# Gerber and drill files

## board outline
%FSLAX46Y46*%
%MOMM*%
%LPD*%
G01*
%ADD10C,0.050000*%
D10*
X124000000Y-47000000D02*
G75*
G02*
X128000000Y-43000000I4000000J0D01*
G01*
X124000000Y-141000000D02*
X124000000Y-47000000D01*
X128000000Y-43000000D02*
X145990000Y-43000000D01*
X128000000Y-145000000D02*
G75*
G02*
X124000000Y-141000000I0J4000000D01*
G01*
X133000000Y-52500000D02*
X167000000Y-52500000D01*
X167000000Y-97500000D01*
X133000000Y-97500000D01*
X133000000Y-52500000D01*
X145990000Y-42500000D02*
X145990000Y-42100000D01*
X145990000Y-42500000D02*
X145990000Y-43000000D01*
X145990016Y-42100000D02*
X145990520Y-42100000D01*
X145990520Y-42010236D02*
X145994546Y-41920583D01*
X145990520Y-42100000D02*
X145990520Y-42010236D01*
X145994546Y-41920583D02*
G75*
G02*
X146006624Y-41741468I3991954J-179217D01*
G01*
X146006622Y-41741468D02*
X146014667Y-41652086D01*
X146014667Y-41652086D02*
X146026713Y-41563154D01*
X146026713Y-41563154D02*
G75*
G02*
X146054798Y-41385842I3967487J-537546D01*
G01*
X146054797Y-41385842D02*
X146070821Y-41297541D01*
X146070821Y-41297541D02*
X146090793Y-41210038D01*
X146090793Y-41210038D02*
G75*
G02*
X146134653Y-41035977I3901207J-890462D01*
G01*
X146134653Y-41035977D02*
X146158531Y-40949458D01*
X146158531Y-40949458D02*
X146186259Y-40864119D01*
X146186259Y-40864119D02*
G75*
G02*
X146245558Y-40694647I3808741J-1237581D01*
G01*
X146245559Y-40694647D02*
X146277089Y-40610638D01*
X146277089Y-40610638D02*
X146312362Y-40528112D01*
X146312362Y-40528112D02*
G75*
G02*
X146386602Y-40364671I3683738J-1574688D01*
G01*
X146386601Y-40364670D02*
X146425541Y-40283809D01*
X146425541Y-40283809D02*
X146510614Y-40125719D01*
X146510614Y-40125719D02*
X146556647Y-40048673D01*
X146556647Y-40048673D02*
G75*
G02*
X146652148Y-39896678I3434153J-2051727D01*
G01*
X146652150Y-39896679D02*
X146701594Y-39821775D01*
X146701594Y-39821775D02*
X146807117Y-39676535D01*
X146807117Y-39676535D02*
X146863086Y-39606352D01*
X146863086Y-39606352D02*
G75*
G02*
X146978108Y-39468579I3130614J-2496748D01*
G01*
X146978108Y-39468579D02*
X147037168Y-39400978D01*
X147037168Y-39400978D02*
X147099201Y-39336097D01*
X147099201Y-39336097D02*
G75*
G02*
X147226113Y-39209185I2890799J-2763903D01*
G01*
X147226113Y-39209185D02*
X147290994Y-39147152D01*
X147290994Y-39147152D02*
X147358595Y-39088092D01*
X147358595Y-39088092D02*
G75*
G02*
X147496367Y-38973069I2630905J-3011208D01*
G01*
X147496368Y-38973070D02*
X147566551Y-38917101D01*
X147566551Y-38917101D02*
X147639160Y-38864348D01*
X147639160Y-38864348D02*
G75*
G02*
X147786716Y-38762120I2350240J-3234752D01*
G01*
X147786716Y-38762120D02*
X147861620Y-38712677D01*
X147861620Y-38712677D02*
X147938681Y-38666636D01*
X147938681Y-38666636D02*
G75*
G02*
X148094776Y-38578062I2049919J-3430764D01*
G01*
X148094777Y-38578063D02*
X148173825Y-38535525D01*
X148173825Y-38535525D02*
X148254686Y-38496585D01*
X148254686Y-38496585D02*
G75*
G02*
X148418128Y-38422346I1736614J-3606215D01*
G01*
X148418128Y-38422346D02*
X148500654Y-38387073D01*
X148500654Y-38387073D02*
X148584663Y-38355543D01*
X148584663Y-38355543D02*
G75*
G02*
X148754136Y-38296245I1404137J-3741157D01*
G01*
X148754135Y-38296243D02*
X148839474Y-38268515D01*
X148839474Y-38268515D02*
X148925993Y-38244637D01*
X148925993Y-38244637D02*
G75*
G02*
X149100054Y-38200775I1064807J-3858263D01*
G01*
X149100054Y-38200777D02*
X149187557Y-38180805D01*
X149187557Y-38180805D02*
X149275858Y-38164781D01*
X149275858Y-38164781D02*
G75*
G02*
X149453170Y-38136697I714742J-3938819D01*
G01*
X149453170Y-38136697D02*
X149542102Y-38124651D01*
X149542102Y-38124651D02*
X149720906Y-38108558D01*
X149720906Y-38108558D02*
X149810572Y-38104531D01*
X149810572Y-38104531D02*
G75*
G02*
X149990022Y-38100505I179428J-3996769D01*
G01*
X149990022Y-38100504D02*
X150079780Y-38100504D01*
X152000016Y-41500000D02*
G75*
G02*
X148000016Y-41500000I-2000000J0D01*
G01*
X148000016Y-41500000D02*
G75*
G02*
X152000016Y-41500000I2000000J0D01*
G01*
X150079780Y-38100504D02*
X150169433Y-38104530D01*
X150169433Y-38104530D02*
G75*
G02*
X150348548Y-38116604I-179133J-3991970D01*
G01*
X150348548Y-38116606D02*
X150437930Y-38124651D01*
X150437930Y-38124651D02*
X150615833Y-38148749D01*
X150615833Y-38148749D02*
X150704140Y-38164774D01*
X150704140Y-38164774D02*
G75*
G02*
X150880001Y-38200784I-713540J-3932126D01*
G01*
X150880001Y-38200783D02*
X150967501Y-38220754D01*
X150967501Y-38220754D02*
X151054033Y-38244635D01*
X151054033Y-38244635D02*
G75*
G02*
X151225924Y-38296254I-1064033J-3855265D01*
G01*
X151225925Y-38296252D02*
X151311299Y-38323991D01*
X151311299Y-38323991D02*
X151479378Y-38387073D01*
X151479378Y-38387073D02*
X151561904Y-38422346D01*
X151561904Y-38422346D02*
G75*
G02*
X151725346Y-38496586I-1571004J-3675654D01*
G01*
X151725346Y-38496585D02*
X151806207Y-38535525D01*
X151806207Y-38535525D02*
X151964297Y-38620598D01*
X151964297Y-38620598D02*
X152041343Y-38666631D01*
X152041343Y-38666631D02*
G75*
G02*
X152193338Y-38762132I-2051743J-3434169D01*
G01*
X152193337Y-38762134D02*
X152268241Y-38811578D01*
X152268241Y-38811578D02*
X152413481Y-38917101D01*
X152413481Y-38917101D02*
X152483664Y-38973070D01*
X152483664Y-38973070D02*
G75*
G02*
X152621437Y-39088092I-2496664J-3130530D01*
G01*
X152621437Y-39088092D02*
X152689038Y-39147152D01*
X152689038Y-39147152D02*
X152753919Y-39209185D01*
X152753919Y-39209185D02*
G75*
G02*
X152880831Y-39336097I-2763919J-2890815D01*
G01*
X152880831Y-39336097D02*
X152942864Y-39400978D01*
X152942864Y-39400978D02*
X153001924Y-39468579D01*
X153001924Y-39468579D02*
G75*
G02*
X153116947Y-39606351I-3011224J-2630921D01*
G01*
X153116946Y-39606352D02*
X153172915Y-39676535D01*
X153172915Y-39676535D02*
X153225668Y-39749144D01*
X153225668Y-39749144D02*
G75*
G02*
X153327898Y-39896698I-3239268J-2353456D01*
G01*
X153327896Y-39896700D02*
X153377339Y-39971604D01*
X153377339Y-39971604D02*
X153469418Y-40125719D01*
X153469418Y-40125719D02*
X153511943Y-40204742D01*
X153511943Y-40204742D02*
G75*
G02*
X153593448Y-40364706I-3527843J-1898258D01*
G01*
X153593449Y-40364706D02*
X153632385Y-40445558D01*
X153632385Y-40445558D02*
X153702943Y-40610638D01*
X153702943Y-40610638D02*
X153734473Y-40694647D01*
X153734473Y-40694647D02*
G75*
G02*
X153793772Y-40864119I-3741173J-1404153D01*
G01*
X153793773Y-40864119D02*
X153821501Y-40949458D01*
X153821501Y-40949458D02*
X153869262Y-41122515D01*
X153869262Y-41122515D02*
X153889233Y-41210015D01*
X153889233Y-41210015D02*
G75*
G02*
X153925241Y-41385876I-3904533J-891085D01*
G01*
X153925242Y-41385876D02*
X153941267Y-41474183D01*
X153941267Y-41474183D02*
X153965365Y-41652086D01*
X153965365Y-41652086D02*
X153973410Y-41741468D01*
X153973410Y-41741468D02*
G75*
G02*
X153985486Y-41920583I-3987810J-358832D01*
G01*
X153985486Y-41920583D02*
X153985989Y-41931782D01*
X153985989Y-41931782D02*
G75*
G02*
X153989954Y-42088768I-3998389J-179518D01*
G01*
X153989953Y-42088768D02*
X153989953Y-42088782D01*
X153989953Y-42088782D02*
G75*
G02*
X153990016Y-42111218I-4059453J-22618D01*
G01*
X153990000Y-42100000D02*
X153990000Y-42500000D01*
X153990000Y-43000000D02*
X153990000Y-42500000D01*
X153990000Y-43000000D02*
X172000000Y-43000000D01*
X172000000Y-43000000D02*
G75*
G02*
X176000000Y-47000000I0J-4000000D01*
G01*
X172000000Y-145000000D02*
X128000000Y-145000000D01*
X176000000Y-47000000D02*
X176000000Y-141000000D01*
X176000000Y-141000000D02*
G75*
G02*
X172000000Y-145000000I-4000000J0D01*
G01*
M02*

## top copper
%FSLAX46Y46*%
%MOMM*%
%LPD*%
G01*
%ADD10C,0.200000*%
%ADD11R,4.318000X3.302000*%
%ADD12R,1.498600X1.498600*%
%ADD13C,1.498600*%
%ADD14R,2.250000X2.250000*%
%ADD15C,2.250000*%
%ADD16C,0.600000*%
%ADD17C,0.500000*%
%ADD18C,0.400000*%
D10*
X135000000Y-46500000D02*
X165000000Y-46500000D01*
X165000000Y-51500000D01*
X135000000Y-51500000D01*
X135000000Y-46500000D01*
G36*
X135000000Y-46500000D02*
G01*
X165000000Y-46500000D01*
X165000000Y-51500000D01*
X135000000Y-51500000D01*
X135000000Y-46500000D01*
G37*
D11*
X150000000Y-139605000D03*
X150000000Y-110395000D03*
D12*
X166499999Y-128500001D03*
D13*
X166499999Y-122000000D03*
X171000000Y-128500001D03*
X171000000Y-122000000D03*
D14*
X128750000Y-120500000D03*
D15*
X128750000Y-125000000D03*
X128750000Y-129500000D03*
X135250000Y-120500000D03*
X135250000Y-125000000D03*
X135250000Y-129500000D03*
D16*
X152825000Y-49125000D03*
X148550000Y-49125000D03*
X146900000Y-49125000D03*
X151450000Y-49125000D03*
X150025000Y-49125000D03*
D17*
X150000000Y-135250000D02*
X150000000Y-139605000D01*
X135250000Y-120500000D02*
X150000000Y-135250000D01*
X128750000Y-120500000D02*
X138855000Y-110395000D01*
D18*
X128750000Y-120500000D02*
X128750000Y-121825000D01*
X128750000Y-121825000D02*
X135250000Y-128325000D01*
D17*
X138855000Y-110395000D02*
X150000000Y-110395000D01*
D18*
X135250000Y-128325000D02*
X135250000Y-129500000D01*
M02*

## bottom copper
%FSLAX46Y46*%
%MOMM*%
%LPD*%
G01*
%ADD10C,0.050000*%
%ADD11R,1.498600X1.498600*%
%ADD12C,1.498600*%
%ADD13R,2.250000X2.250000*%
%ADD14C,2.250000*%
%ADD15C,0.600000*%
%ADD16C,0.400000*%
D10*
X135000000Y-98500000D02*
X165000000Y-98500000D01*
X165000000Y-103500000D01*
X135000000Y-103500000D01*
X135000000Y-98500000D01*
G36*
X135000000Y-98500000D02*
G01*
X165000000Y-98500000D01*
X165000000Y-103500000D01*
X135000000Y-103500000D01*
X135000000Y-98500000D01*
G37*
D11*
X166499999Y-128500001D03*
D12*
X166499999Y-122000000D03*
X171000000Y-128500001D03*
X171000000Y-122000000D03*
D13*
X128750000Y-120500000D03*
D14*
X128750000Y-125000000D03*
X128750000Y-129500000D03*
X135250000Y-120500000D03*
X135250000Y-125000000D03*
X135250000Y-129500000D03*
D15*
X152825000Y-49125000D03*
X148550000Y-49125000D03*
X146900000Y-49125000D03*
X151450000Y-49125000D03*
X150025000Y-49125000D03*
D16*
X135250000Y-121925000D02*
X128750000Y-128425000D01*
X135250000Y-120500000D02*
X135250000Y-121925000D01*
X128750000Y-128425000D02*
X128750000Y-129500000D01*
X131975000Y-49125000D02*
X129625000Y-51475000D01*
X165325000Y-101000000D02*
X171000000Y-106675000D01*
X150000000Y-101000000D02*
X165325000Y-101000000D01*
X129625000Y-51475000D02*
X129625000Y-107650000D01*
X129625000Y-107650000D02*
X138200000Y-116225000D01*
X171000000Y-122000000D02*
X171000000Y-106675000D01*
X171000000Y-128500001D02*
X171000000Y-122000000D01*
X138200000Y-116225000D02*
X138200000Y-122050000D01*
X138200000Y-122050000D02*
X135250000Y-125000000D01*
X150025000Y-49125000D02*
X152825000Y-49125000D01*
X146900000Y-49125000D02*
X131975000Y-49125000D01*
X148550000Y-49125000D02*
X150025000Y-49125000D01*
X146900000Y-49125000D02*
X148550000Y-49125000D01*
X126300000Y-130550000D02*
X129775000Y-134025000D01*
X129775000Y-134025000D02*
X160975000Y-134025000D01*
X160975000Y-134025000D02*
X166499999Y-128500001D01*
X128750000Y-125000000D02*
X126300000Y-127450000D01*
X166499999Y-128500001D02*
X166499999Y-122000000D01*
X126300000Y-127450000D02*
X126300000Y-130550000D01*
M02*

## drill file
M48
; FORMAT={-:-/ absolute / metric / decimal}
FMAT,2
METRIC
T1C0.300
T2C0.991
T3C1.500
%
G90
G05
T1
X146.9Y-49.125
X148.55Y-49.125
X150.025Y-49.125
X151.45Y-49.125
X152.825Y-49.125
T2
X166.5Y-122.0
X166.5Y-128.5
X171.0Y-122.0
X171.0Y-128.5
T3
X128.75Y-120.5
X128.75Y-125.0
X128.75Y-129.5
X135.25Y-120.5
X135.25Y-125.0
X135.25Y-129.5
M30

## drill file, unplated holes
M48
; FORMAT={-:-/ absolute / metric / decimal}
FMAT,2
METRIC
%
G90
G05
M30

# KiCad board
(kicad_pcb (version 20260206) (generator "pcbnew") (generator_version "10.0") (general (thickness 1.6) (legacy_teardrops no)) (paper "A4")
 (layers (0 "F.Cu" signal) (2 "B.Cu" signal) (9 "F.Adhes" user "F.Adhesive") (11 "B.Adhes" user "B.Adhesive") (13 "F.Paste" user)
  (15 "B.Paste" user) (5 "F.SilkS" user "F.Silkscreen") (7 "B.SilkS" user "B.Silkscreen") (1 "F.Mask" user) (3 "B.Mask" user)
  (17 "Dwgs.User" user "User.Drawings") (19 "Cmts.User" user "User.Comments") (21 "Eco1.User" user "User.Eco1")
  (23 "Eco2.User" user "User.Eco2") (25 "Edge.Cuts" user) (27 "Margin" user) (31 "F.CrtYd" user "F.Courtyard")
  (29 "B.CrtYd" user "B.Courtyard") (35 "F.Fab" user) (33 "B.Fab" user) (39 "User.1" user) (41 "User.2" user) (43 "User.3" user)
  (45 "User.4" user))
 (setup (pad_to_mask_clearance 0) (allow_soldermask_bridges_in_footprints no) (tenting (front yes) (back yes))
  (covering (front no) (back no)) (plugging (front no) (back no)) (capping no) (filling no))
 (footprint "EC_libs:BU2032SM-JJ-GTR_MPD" (layer "F.Cu") (at 150 125 -90)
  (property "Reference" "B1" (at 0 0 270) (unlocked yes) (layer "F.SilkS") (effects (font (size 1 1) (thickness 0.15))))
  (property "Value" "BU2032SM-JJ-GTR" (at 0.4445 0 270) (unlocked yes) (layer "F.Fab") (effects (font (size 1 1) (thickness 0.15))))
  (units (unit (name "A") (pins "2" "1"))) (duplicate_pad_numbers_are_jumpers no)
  (pad "1" smd rect (at 14.605 0 270) (size 3.302 4.318) (layers "F.Cu" "F.Mask" "F.Paste") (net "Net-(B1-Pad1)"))
  (pad "2" smd rect (at -14.605 0 270) (size 3.302 4.318) (layers "F.Cu" "F.Mask" "F.Paste") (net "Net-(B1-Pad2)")))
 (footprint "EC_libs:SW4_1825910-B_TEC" (layer "F.Cu") (at 171 122 90)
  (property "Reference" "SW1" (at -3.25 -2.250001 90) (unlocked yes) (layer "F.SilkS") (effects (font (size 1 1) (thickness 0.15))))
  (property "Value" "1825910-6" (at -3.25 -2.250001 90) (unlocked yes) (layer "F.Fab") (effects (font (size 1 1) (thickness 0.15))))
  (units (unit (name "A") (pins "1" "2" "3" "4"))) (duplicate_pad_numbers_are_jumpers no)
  (pad "1" thru_hole rect (at -6.500001 -4.500001 90) (size 1.4986 1.4986) (drill 0.9906) (layers "*.Cu" "*.Mask") (remove_unused_layers no)
   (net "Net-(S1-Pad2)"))
  (pad "2" thru_hole circle (at 0 -4.500001 90) (size 1.4986 1.4986) (drill 0.9906) (layers "*.Cu" "*.Mask") (remove_unused_layers no)
   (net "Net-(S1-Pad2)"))
  (pad "3" thru_hole circle (at -6.500001 0 90) (size 1.4986 1.4986) (drill 0.9906) (layers "*.Cu" "*.Mask") (remove_unused_layers no)
   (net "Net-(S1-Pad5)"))
  (pad "4" thru_hole circle (at 0 0 90) (size 1.4986 1.4986) (drill 0.9906) (layers "*.Cu" "*.Mask") (remove_unused_layers no)
   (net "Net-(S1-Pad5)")))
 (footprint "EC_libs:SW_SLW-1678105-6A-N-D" (layer "F.Cu") (at 132 125 -90)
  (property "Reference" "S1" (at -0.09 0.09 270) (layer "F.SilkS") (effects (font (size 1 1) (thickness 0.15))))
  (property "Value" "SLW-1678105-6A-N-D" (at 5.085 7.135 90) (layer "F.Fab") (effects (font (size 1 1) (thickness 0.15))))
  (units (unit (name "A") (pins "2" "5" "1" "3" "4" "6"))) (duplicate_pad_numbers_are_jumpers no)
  (pad "1" thru_hole rect (at -4.5 3.25 270) (size 2.25 2.25) (drill 1.5) (layers "*.Cu" "*.Mask") (remove_unused_layers no)
   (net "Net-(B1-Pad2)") (solder_mask_margin 0.102))
  (pad "2" thru_hole circle (at 0 3.25 270) (size 2.25 2.25) (drill 1.5) (layers "*.Cu" "*.Mask") (remove_unused_layers no)
   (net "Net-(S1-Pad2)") (solder_mask_margin 0.102))
  (pad "3" thru_hole circle (at 4.5 3.25 270) (size 2.25 2.25) (drill 1.5) (layers "*.Cu" "*.Mask") (remove_unused_layers no)
   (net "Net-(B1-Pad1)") (solder_mask_margin 0.102))
  (pad "4" thru_hole circle (at -4.5 -3.25 270) (size 2.25 2.25) (drill 1.5) (layers "*.Cu" "*.Mask") (remove_unused_layers no)
   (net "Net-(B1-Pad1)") (solder_mask_margin 0.102))
  (pad "5" thru_hole circle (at 0 -3.25 270) (size 2.25 2.25) (drill 1.5) (layers "*.Cu" "*.Mask") (remove_unused_layers no)
   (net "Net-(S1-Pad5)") (solder_mask_margin 0.102))
  (pad "6" thru_hole circle (at 4.5 -3.25 270) (size 2.25 2.25) (drill 1.5) (layers "*.Cu" "*.Mask") (remove_unused_layers no)
   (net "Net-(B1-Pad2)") (solder_mask_margin 0.102)))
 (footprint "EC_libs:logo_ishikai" (layer "F.Cu") (at 168.51 109.35)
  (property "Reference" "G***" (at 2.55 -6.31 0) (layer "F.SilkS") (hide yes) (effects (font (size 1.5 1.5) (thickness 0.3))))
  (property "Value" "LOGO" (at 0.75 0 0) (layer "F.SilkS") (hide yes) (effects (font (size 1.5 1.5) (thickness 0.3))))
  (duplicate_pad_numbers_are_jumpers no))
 (gr_rect (start 135 46.5) (end 165 51.5) (stroke (width 0.2) (type solid)) (fill yes) (layer "F.Cu") (net "Net-(S1-Pad5)"))
 (gr_rect (start 135 98.5) (end 165 103.5) (stroke (width 0.05) (type solid)) (fill yes) (layer "B.Cu") (net "Net-(S1-Pad5)"))
 (gr_arc (start 124 47) (mid 125.171573 44.171573) (end 128 43) (stroke (width 0.05) (type default)) (layer "Edge.Cuts"))
 (gr_line (start 124 141) (end 124 47) (stroke (width 0.05) (type default)) (layer "Edge.Cuts"))
 (gr_line (start 128 43) (end 145.99 43) (stroke (width 0.05) (type default)) (layer "Edge.Cuts"))
 (gr_arc (start 128 145) (mid 125.171573 143.828427) (end 124 141) (stroke (width 0.05) (type default)) (layer "Edge.Cuts"))
 (gr_rect (start 133 52.5) (end 167 97.5) (stroke (width 0.05) (type solid)) (fill no) (layer "Edge.Cuts"))
 (gr_line (start 145.99 42.5) (end 145.99 42.1) (stroke (width 0.05) (type default)) (layer "Edge.Cuts"))
 (gr_line (start 145.99 42.5) (end 145.99 43) (stroke (width 0.05) (type default)) (layer "Edge.Cuts"))
 (gr_line (start 145.990016 42.1) (end 145.99052 42.1) (stroke (width 0.05) (type default)) (layer "Edge.Cuts"))
 (gr_line (start 145.99052 42.010236) (end 145.994546 41.920583) (stroke (width 0.05) (type default)) (layer "Edge.Cuts"))
 (gr_line (start 145.99052 42.1) (end 145.99052 42.010236) (stroke (width 0.05) (type default)) (layer "Edge.Cuts"))
 (gr_arc (start 145.994546 41.920583) (mid 145.999578 41.830958) (end 146.006622 41.741468) (stroke (width 0.05) (type default))
  (layer "Edge.Cuts"))
 (gr_line (start 146.006622 41.741468) (end 146.014667 41.652086) (stroke (width 0.05) (type default)) (layer "Edge.Cuts"))
 (gr_line (start 146.014667 41.652086) (end 146.026713 41.563154) (stroke (width 0.05) (type default)) (layer "Edge.Cuts"))
 (gr_arc (start 146.026713 41.563154) (mid 146.039761 41.474341) (end 146.054797 41.385842) (stroke (width 0.05) (type default))
  (layer "Edge.Cuts"))
 (gr_line (start 146.054797 41.385842) (end 146.070821 41.297541) (stroke (width 0.05) (type default)) (layer "Edge.Cuts"))
 (gr_line (start 146.070821 41.297541) (end 146.090793 41.210038) (stroke (width 0.05) (type default)) (layer "Edge.Cuts"))
 (gr_arc (start 146.090793 41.210038) (mid 146.111747 41.122761) (end 146.134653 41.035977) (stroke (width 0.05) (type default))
  (layer "Edge.Cuts"))
 (gr_line (start 146.134653 41.035977) (end 146.158531 40.949458) (stroke (width 0.05) (type default)) (layer "Edge.Cuts"))
 (gr_line (start 146.158531 40.949458) (end 146.186259 40.864119) (stroke (width 0.05) (type default)) (layer "Edge.Cuts"))
 (gr_arc (start 146.186259 40.864119) (mid 146.214959 40.779051) (end 146.245559 40.694647) (stroke (width 0.05) (type default))
  (layer "Edge.Cuts"))
 (gr_line (start 146.245559 40.694647) (end 146.277089 40.610638) (stroke (width 0.05) (type default)) (layer "Edge.Cuts"))
 (gr_line (start 146.277089 40.610638) (end 146.312362 40.528112) (stroke (width 0.05) (type default)) (layer "Edge.Cuts"))
 (gr_arc (start 146.312362 40.528112) (mid 146.348566 40.445975) (end 146.386601 40.36467) (stroke (width 0.05) (type default))
  (layer "Edge.Cuts"))
 (gr_line (start 146.386601 40.36467) (end 146.425541 40.283809) (stroke (width 0.05) (type default)) (layer "Edge.Cuts"))
 (gr_line (start 146.425541 40.283809) (end 146.510614 40.125719) (stroke (width 0.05) (type default)) (layer "Edge.Cuts"))
 (gr_line (start 146.510614 40.125719) (end 146.556647 40.048673) (stroke (width 0.05) (type default)) (layer "Edge.Cuts"))
 (gr_arc (start 146.556647 40.048673) (mid 146.603546 39.97214) (end 146.65215 39.896679) (stroke (width 0.05) (type default))
  (layer "Edge.Cuts"))
 (gr_line (start 146.65215 39.896679) (end 146.701594 39.821775) (stroke (width 0.05) (type default)) (layer "Edge.Cuts"))
 (gr_line (start 146.701594 39.821775) (end 146.807117 39.676535) (stroke (width 0.05) (type default)) (layer "Edge.Cuts"))
 (gr_line (start 146.807117 39.676535) (end 146.863086 39.606352) (stroke (width 0.05) (type default)) (layer "Edge.Cuts"))
 (gr_arc (start 146.863086 39.606352) (mid 146.919825 39.536821) (end 146.978108 39.468579) (stroke (width 0.05) (type default))
  (layer "Edge.Cuts"))
 (gr_line (start 146.978108 39.468579) (end 147.037168 39.400978) (stroke (width 0.05) (type default)) (layer "Edge.Cuts"))
 (gr_line (start 147.037168 39.400978) (end 147.099201 39.336097) (stroke (width 0.05) (type default)) (layer "Edge.Cuts"))
 (gr_arc (start 147.099201 39.336097) (mid 147.161945 39.271929) (end 147.226113 39.209185) (stroke (width 0.05) (type default))
  (layer "Edge.Cuts"))
 (gr_line (start 147.226113 39.209185) (end 147.290994 39.147152) (stroke (width 0.05) (type default)) (layer "Edge.Cuts"))
 (gr_line (start 147.290994 39.147152) (end 147.358595 39.088092) (stroke (width 0.05) (type default)) (layer "Edge.Cuts"))
 (gr_arc (start 147.358595 39.088092) (mid 147.426836 39.029808) (end 147.496368 38.97307) (stroke (width 0.05) (type default))
  (layer "Edge.Cuts"))
 (gr_line (start 147.496368 38.97307) (end 147.566551 38.917101) (stroke (width 0.05) (type default)) (layer "Edge.Cuts"))
 (gr_line (start 147.566551 38.917101) (end 147.63916 38.864348) (stroke (width 0.05) (type default)) (layer "Edge.Cuts"))
 (gr_arc (start 147.63916 38.864348) (mid 147.712364 38.812406) (end 147.786716 38.76212) (stroke (width 0.05) (type default))
  (layer "Edge.Cuts"))
 (gr_line (start 147.786716 38.76212) (end 147.86162 38.712677) (stroke (width 0.05) (type default)) (layer "Edge.Cuts"))
 (gr_line (start 147.86162 38.712677) (end 147.938681 38.666636) (stroke (width 0.05) (type default)) (layer "Edge.Cuts"))
 (gr_arc (start 147.938681 38.666636) (mid 148.016232 38.621473) (end 148.094777 38.578063) (stroke (width 0.05) (type default))
  (layer "Edge.Cuts"))
 (gr_line (start 148.094777 38.578063) (end 148.173825 38.535525) (stroke (width 0.05) (type default)) (layer "Edge.Cuts"))
 (gr_line (start 148.173825 38.535525) (end 148.254686 38.496585) (stroke (width 0.05) (type default)) (layer "Edge.Cuts"))
 (gr_arc (start 148.254686 38.496585) (mid 148.335991 38.458549) (end 148.418128 38.422346) (stroke (width 0.05) (type default))
  (layer "Edge.Cuts"))
 (gr_line (start 148.418128 38.422346) (end 148.500654 38.387073) (stroke (width 0.05) (type default)) (layer "Edge.Cuts"))
 (gr_line (start 148.500654 38.387073) (end 148.584663 38.355543) (stroke (width 0.05) (type default)) (layer "Edge.Cuts"))
 (gr_arc (start 148.584663 38.355543) (mid 148.669066 38.324941) (end 148.754135 38.296243) (stroke (width 0.05) (type default))
  (layer "Edge.Cuts"))
 (gr_line (start 148.754135 38.296243) (end 148.839474 38.268515) (stroke (width 0.05) (type default)) (layer "Edge.Cuts"))
 (gr_line (start 148.839474 38.268515) (end 148.925993 38.244637) (stroke (width 0.05) (type default)) (layer "Edge.Cuts"))
 (gr_arc (start 148.925993 38.244637) (mid 149.012778 38.221731) (end 149.100054 38.200777) (stroke (width 0.05) (type default))
  (layer "Edge.Cuts"))
 (gr_line (start 149.100054 38.200777) (end 149.187557 38.180805) (stroke (width 0.05) (type default)) (layer "Edge.Cuts"))
 (gr_line (start 149.187557 38.180805) (end 149.275858 38.164781) (stroke (width 0.05) (type default)) (layer "Edge.Cuts"))
 (gr_arc (start 149.275858 38.164781) (mid 149.364356 38.149745) (end 149.45317 38.136697) (stroke (width 0.05) (type default))
  (layer "Edge.Cuts"))
 (gr_line (start 149.45317 38.136697) (end 149.542102 38.124651) (stroke (width 0.05) (type default)) (layer "Edge.Cuts"))
 (gr_line (start 149.542102 38.124651) (end 149.720906 38.108558) (stroke (width 0.05) (type default)) (layer "Edge.Cuts"))
 (gr_line (start 149.720906 38.108558) (end 149.810572 38.104531) (stroke (width 0.05) (type default)) (layer "Edge.Cuts"))
 (gr_arc (start 149.810572 38.104531) (mid 149.900274 38.101511) (end 149.990022 38.100504) (stroke (width 0.05) (type default))
  (layer "Edge.Cuts"))
 (gr_line (start 149.990022 38.100504) (end 150.07978 38.100504) (stroke (width 0.05) (type default)) (layer "Edge.Cuts"))
 (gr_circle (center 150.000016 41.5) (end 152.000016 41.5) (stroke (width 0.05) (type solid)) (fill no) (layer "Edge.Cuts"))
 (gr_line (start 150.07978 38.100504) (end 150.169433 38.10453) (stroke (width 0.05) (type default)) (layer "Edge.Cuts"))
 (gr_arc (start 150.169433 38.10453) (mid 150.259058 38.109562) (end 150.348548 38.116606) (stroke (width 0.05) (type default))
  (layer "Edge.Cuts"))
 (gr_line (start 150.348548 38.116606) (end 150.43793 38.124651) (stroke (width 0.05) (type default)) (layer "Edge.Cuts"))
 (gr_line (start 150.43793 38.124651) (end 150.615833 38.148749) (stroke (width 0.05) (type default)) (layer "Edge.Cuts"))
 (gr_line (start 150.615833 38.148749) (end 150.70414 38.164774) (stroke (width 0.05) (type default)) (layer "Edge.Cuts"))
 (gr_arc (start 150.70414 38.164774) (mid 150.792273 38.181791) (end 150.880001 38.200783) (stroke (width 0.05) (type default))
  (layer "Edge.Cuts"))
 (gr_line (start 150.880001 38.200783) (end 150.967501 38.220754) (stroke (width 0.05) (type default)) (layer "Edge.Cuts"))
 (gr_line (start 150.967501 38.220754) (end 151.054033 38.244635) (stroke (width 0.05) (type default)) (layer "Edge.Cuts"))
 (gr_arc (start 151.054033 38.244635) (mid 151.140268 38.269479) (end 151.225925 38.296252) (stroke (width 0.05) (type default))
  (layer "Edge.Cuts"))
 (gr_line (start 151.225925 38.296252) (end 151.311299 38.323991) (stroke (width 0.05) (type default)) (layer "Edge.Cuts"))
 (gr_line (start 151.311299 38.323991) (end 151.479378 38.387073) (stroke (width 0.05) (type default)) (layer "Edge.Cuts"))
 (gr_line (start 151.479378 38.387073) (end 151.561904 38.422346) (stroke (width 0.05) (type default)) (layer "Edge.Cuts"))
 (gr_arc (start 151.561904 38.422346) (mid 151.644042 38.458548) (end 151.725346 38.496585) (stroke (width 0.05) (type default))
  (layer "Edge.Cuts"))
 (gr_line (start 151.725346 38.496585) (end 151.806207 38.535525) (stroke (width 0.05) (type default)) (layer "Edge.Cuts"))
 (gr_line (start 151.806207 38.535525) (end 151.964297 38.620598) (stroke (width 0.05) (type default)) (layer "Edge.Cuts"))
 (gr_line (start 151.964297 38.620598) (end 152.041343 38.666631) (stroke (width 0.05) (type default)) (layer "Edge.Cuts"))
 (gr_arc (start 152.041343 38.666631) (mid 152.117876 38.71353) (end 152.193337 38.762134) (stroke (width 0.05) (type default))
  (layer "Edge.Cuts"))
 (gr_line (start 152.193337 38.762134) (end 152.268241 38.811578) (stroke (width 0.05) (type default)) (layer "Edge.Cuts"))
 (gr_line (start 152.268241 38.811578) (end 152.413481 38.917101) (stroke (width 0.05) (type default)) (layer "Edge.Cuts"))
 (gr_line (start 152.413481 38.917101) (end 152.483664 38.97307) (stroke (width 0.05) (type default)) (layer "Edge.Cuts"))
 (gr_arc (start 152.483664 38.97307) (mid 152.553195 39.029809) (end 152.621437 39.088092) (stroke (width 0.05) (type default))
  (layer "Edge.Cuts"))
 (gr_line (start 152.621437 39.088092) (end 152.689038 39.147152) (stroke (width 0.05) (type default)) (layer "Edge.Cuts"))
 (gr_line (start 152.689038 39.147152) (end 152.753919 39.209185) (stroke (width 0.05) (type default)) (layer "Edge.Cuts"))
 (gr_arc (start 152.753919 39.209185) (mid 152.818087 39.271929) (end 152.880831 39.336097) (stroke (width 0.05) (type default))
  (layer "Edge.Cuts"))
 (gr_line (start 152.880831 39.336097) (end 152.942864 39.400978) (stroke (width 0.05) (type default)) (layer "Edge.Cuts"))
 (gr_line (start 152.942864 39.400978) (end 153.001924 39.468579) (stroke (width 0.05) (type default)) (layer "Edge.Cuts"))
 (gr_arc (start 153.001924 39.468579) (mid 153.060208 39.53682) (end 153.116946 39.606352) (stroke (width 0.05) (type default))
  (layer "Edge.Cuts"))
 (gr_line (start 153.116946 39.606352) (end 153.172915 39.676535) (stroke (width 0.05) (type default)) (layer "Edge.Cuts"))
 (gr_line (start 153.172915 39.676535) (end 153.225668 39.749144) (stroke (width 0.05) (type default)) (layer "Edge.Cuts"))
 (gr_arc (start 153.225668 39.749144) (mid 153.277609 39.822349) (end 153.327896 39.8967) (stroke (width 0.05) (type default))
  (layer "Edge.Cuts"))
 (gr_line (start 153.327896 39.8967) (end 153.377339 39.971604) (stroke (width 0.05) (type default)) (layer "Edge.Cuts"))
 (gr_line (start 153.377339 39.971604) (end 153.469418 40.125719) (stroke (width 0.05) (type default)) (layer "Edge.Cuts"))
 (gr_line (start 153.469418 40.125719) (end 153.511943 40.204742) (stroke (width 0.05) (type default)) (layer "Edge.Cuts"))
 (gr_arc (start 153.511943 40.204742) (mid 153.553592 40.284267) (end 153.593449 40.364706) (stroke (width 0.05) (type default))
  (layer "Edge.Cuts"))
 (gr_line (start 153.593449 40.364706) (end 153.632385 40.445558) (stroke (width 0.05) (type default)) (layer "Edge.Cuts"))
 (gr_line (start 153.632385 40.445558) (end 153.702943 40.610638) (stroke (width 0.05) (type default)) (layer "Edge.Cuts"))
 (gr_line (start 153.702943 40.610638) (end 153.734473 40.694647) (stroke (width 0.05) (type default)) (layer "Edge.Cuts"))
 (gr_arc (start 153.734473 40.694647) (mid 153.765075 40.77905) (end 153.793773 40.864119) (stroke (width 0.05) (type default))
  (layer "Edge.Cuts"))
 (gr_line (start 153.793773 40.864119) (end 153.821501 40.949458) (stroke (width 0.05) (type default)) (layer "Edge.Cuts"))
 (gr_line (start 153.821501 40.949458) (end 153.869262 41.122515) (stroke (width 0.05) (type default)) (layer "Edge.Cuts"))
 (gr_line (start 153.869262 41.122515) (end 153.889233 41.210015) (stroke (width 0.05) (type default)) (layer "Edge.Cuts"))
 (gr_arc (start 153.889233 41.210015) (mid 153.908223 41.297744) (end 153.925242 41.385876) (stroke (width 0.05) (type default))
  (layer "Edge.Cuts"))
 (gr_line (start 153.925242 41.385876) (end 153.941267 41.474183) (stroke (width 0.05) (type default)) (layer "Edge.Cuts"))
 (gr_line (start 153.941267 41.474183) (end 153.965365 41.652086) (stroke (width 0.05) (type default)) (layer "Edge.Cuts"))
 (gr_line (start 153.965365 41.652086) (end 153.97341 41.741468) (stroke (width 0.05) (type default)) (layer "Edge.Cuts"))
 (gr_arc (start 153.97341 41.741468) (mid 153.980452 41.830958) (end 153.985486 41.920583) (stroke (width 0.05) (type default))
  (layer "Edge.Cuts"))
 (gr_line (start 153.985486 41.920583) (end 153.985989 41.931782) (stroke (width 0.05) (type default)) (layer "Edge.Cuts"))
 (gr_arc (start 153.985989 41.931782) (mid 153.988741 42.010256) (end 153.989953 42.088768) (stroke (width 0.05) (type default))
  (layer "Edge.Cuts"))
 (gr_line (start 153.989953 42.088768) (end 153.989953 42.088782) (stroke (width 0.05) (type default)) (layer "Edge.Cuts"))
 (gr_arc (start 153.989953 42.088782) (mid 153.99 42.1) (end 153.990016 42.111218) (stroke (width 0.05) (type default)) (layer "Edge.Cuts"))
 (gr_line (start 153.99 42.1) (end 153.99 42.5) (stroke (width 0.05) (type default)) (layer "Edge.Cuts"))
 (gr_line (start 153.99 43) (end 153.99 42.5) (stroke (width 0.05) (type default)) (layer "Edge.Cuts"))
 (gr_line (start 153.99 43) (end 172 43) (stroke (width 0.05) (type default)) (layer "Edge.Cuts"))
 (gr_arc (start 172 43) (mid 174.828427 44.171573) (end 176 47) (stroke (width 0.05) (type default)) (layer "Edge.Cuts"))
 (gr_line (start 172 145) (end 128 145) (stroke (width 0.05) (type default)) (layer "Edge.Cuts"))
 (gr_line (start 176 47) (end 176 141) (stroke (width 0.05) (type default)) (layer "Edge.Cuts"))
 (gr_arc (start 176 141) (mid 174.828427 143.828427) (end 172 145) (stroke (width 0.05) (type default)) (layer "Edge.Cuts"))
 (segment (start 150 135.25) (end 150 139.605) (width 0.5) (layer "F.Cu") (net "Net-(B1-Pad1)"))
 (segment (start 135.25 120.5) (end 150 135.25) (width 0.5) (layer "F.Cu") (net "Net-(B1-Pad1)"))
 (segment (start 135.25 121.925) (end 128.75 128.425) (width 0.4) (layer "B.Cu") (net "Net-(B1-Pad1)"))
 (segment (start 135.25 120.5) (end 135.25 121.925) (width 0.4) (layer "B.Cu") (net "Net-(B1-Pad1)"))
 (segment (start 128.75 128.425) (end 128.75 129.5) (width 0.4) (layer "B.Cu") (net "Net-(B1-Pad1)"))
 (segment (start 128.75 120.5) (end 138.855 110.395) (width 0.5) (layer "F.Cu") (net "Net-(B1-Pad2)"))
 (segment (start 128.75 120.5) (end 128.75 121.825) (width 0.4) (layer "F.Cu") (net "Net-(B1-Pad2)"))
 (segment (start 128.75 121.825) (end 135.25 128.325) (width 0.4) (layer "F.Cu") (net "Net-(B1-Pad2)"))
 (segment (start 138.855 110.395) (end 150 110.395) (width 0.5) (layer "F.Cu") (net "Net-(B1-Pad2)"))
 (segment (start 135.25 128.325) (end 135.25 129.5) (width 0.4) (layer "F.Cu") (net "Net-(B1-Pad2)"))
 (segment (start 126.3 130.55) (end 129.775 134.025) (width 0.4) (layer "B.Cu") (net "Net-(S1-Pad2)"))
 (segment (start 129.775 134.025) (end 160.975 134.025) (width 0.4) (layer "B.Cu") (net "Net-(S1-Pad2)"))
 (segment (start 160.975 134.025) (end 166.499999 128.500001) (width 0.4) (layer "B.Cu") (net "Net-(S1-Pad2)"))
 (segment (start 128.75 125) (end 126.3 127.45) (width 0.4) (layer "B.Cu") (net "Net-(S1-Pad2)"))
 (segment (start 166.499999 128.500001) (end 166.499999 122) (width 0.4) (layer "B.Cu") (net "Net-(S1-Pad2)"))
 (segment (start 126.3 127.45) (end 126.3 130.55) (width 0.4) (layer "B.Cu") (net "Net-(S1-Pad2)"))
 (via (at 152.825 49.125) (size 0.6) (drill 0.3) (layers "F.Cu" "B.Cu") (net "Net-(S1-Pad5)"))
 (via (at 148.55 49.125) (size 0.6) (drill 0.3) (layers "F.Cu" "B.Cu") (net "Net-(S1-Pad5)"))
 (via (at 146.9 49.125) (size 0.6) (drill 0.3) (layers "F.Cu" "B.Cu") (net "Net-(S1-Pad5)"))
 (via (at 151.45 49.125) (size 0.6) (drill 0.3) (layers "F.Cu" "B.Cu") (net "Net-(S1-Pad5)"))
 (via (at 150.025 49.125) (size 0.6) (drill 0.3) (layers "F.Cu" "B.Cu") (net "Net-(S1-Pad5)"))
 (segment (start 131.975 49.125) (end 129.625 51.475) (width 0.4) (layer "B.Cu") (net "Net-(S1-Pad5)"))
 (segment (start 165.325 101) (end 171 106.675) (width 0.4) (layer "B.Cu") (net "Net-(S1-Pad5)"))
 (segment (start 150 101) (end 165.325 101) (width 0.4) (layer "B.Cu") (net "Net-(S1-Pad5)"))
 (segment (start 129.625 51.475) (end 129.625 107.65) (width 0.4) (layer "B.Cu") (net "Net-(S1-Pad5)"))
 (segment (start 129.625 107.65) (end 138.2 116.225) (width 0.4) (layer "B.Cu") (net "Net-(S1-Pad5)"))
 (segment (start 171 122) (end 171 106.675) (width 0.4) (layer "B.Cu") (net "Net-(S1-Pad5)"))
 (segment (start 171 128.500001) (end 171 122) (width 0.4) (layer "B.Cu") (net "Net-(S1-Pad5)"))
 (segment (start 138.2 116.225) (end 138.2 122.05) (width 0.4) (layer "B.Cu") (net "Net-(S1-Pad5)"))
 (segment (start 138.2 122.05) (end 135.25 125) (width 0.4) (layer "B.Cu") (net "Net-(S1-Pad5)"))
 (segment (start 150.025 49.125) (end 152.825 49.125) (width 0.4) (layer "B.Cu") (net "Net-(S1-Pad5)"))
 (segment (start 146.9 49.125) (end 131.975 49.125) (width 0.4) (layer "B.Cu") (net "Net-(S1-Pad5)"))
 (segment (start 148.55 49.125) (end 150.025 49.125) (width 0.4) (layer "B.Cu") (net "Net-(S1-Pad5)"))
 (segment (start 146.9 49.125) (end 148.55 49.125) (width 0.4) (layer "B.Cu") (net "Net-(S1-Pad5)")))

